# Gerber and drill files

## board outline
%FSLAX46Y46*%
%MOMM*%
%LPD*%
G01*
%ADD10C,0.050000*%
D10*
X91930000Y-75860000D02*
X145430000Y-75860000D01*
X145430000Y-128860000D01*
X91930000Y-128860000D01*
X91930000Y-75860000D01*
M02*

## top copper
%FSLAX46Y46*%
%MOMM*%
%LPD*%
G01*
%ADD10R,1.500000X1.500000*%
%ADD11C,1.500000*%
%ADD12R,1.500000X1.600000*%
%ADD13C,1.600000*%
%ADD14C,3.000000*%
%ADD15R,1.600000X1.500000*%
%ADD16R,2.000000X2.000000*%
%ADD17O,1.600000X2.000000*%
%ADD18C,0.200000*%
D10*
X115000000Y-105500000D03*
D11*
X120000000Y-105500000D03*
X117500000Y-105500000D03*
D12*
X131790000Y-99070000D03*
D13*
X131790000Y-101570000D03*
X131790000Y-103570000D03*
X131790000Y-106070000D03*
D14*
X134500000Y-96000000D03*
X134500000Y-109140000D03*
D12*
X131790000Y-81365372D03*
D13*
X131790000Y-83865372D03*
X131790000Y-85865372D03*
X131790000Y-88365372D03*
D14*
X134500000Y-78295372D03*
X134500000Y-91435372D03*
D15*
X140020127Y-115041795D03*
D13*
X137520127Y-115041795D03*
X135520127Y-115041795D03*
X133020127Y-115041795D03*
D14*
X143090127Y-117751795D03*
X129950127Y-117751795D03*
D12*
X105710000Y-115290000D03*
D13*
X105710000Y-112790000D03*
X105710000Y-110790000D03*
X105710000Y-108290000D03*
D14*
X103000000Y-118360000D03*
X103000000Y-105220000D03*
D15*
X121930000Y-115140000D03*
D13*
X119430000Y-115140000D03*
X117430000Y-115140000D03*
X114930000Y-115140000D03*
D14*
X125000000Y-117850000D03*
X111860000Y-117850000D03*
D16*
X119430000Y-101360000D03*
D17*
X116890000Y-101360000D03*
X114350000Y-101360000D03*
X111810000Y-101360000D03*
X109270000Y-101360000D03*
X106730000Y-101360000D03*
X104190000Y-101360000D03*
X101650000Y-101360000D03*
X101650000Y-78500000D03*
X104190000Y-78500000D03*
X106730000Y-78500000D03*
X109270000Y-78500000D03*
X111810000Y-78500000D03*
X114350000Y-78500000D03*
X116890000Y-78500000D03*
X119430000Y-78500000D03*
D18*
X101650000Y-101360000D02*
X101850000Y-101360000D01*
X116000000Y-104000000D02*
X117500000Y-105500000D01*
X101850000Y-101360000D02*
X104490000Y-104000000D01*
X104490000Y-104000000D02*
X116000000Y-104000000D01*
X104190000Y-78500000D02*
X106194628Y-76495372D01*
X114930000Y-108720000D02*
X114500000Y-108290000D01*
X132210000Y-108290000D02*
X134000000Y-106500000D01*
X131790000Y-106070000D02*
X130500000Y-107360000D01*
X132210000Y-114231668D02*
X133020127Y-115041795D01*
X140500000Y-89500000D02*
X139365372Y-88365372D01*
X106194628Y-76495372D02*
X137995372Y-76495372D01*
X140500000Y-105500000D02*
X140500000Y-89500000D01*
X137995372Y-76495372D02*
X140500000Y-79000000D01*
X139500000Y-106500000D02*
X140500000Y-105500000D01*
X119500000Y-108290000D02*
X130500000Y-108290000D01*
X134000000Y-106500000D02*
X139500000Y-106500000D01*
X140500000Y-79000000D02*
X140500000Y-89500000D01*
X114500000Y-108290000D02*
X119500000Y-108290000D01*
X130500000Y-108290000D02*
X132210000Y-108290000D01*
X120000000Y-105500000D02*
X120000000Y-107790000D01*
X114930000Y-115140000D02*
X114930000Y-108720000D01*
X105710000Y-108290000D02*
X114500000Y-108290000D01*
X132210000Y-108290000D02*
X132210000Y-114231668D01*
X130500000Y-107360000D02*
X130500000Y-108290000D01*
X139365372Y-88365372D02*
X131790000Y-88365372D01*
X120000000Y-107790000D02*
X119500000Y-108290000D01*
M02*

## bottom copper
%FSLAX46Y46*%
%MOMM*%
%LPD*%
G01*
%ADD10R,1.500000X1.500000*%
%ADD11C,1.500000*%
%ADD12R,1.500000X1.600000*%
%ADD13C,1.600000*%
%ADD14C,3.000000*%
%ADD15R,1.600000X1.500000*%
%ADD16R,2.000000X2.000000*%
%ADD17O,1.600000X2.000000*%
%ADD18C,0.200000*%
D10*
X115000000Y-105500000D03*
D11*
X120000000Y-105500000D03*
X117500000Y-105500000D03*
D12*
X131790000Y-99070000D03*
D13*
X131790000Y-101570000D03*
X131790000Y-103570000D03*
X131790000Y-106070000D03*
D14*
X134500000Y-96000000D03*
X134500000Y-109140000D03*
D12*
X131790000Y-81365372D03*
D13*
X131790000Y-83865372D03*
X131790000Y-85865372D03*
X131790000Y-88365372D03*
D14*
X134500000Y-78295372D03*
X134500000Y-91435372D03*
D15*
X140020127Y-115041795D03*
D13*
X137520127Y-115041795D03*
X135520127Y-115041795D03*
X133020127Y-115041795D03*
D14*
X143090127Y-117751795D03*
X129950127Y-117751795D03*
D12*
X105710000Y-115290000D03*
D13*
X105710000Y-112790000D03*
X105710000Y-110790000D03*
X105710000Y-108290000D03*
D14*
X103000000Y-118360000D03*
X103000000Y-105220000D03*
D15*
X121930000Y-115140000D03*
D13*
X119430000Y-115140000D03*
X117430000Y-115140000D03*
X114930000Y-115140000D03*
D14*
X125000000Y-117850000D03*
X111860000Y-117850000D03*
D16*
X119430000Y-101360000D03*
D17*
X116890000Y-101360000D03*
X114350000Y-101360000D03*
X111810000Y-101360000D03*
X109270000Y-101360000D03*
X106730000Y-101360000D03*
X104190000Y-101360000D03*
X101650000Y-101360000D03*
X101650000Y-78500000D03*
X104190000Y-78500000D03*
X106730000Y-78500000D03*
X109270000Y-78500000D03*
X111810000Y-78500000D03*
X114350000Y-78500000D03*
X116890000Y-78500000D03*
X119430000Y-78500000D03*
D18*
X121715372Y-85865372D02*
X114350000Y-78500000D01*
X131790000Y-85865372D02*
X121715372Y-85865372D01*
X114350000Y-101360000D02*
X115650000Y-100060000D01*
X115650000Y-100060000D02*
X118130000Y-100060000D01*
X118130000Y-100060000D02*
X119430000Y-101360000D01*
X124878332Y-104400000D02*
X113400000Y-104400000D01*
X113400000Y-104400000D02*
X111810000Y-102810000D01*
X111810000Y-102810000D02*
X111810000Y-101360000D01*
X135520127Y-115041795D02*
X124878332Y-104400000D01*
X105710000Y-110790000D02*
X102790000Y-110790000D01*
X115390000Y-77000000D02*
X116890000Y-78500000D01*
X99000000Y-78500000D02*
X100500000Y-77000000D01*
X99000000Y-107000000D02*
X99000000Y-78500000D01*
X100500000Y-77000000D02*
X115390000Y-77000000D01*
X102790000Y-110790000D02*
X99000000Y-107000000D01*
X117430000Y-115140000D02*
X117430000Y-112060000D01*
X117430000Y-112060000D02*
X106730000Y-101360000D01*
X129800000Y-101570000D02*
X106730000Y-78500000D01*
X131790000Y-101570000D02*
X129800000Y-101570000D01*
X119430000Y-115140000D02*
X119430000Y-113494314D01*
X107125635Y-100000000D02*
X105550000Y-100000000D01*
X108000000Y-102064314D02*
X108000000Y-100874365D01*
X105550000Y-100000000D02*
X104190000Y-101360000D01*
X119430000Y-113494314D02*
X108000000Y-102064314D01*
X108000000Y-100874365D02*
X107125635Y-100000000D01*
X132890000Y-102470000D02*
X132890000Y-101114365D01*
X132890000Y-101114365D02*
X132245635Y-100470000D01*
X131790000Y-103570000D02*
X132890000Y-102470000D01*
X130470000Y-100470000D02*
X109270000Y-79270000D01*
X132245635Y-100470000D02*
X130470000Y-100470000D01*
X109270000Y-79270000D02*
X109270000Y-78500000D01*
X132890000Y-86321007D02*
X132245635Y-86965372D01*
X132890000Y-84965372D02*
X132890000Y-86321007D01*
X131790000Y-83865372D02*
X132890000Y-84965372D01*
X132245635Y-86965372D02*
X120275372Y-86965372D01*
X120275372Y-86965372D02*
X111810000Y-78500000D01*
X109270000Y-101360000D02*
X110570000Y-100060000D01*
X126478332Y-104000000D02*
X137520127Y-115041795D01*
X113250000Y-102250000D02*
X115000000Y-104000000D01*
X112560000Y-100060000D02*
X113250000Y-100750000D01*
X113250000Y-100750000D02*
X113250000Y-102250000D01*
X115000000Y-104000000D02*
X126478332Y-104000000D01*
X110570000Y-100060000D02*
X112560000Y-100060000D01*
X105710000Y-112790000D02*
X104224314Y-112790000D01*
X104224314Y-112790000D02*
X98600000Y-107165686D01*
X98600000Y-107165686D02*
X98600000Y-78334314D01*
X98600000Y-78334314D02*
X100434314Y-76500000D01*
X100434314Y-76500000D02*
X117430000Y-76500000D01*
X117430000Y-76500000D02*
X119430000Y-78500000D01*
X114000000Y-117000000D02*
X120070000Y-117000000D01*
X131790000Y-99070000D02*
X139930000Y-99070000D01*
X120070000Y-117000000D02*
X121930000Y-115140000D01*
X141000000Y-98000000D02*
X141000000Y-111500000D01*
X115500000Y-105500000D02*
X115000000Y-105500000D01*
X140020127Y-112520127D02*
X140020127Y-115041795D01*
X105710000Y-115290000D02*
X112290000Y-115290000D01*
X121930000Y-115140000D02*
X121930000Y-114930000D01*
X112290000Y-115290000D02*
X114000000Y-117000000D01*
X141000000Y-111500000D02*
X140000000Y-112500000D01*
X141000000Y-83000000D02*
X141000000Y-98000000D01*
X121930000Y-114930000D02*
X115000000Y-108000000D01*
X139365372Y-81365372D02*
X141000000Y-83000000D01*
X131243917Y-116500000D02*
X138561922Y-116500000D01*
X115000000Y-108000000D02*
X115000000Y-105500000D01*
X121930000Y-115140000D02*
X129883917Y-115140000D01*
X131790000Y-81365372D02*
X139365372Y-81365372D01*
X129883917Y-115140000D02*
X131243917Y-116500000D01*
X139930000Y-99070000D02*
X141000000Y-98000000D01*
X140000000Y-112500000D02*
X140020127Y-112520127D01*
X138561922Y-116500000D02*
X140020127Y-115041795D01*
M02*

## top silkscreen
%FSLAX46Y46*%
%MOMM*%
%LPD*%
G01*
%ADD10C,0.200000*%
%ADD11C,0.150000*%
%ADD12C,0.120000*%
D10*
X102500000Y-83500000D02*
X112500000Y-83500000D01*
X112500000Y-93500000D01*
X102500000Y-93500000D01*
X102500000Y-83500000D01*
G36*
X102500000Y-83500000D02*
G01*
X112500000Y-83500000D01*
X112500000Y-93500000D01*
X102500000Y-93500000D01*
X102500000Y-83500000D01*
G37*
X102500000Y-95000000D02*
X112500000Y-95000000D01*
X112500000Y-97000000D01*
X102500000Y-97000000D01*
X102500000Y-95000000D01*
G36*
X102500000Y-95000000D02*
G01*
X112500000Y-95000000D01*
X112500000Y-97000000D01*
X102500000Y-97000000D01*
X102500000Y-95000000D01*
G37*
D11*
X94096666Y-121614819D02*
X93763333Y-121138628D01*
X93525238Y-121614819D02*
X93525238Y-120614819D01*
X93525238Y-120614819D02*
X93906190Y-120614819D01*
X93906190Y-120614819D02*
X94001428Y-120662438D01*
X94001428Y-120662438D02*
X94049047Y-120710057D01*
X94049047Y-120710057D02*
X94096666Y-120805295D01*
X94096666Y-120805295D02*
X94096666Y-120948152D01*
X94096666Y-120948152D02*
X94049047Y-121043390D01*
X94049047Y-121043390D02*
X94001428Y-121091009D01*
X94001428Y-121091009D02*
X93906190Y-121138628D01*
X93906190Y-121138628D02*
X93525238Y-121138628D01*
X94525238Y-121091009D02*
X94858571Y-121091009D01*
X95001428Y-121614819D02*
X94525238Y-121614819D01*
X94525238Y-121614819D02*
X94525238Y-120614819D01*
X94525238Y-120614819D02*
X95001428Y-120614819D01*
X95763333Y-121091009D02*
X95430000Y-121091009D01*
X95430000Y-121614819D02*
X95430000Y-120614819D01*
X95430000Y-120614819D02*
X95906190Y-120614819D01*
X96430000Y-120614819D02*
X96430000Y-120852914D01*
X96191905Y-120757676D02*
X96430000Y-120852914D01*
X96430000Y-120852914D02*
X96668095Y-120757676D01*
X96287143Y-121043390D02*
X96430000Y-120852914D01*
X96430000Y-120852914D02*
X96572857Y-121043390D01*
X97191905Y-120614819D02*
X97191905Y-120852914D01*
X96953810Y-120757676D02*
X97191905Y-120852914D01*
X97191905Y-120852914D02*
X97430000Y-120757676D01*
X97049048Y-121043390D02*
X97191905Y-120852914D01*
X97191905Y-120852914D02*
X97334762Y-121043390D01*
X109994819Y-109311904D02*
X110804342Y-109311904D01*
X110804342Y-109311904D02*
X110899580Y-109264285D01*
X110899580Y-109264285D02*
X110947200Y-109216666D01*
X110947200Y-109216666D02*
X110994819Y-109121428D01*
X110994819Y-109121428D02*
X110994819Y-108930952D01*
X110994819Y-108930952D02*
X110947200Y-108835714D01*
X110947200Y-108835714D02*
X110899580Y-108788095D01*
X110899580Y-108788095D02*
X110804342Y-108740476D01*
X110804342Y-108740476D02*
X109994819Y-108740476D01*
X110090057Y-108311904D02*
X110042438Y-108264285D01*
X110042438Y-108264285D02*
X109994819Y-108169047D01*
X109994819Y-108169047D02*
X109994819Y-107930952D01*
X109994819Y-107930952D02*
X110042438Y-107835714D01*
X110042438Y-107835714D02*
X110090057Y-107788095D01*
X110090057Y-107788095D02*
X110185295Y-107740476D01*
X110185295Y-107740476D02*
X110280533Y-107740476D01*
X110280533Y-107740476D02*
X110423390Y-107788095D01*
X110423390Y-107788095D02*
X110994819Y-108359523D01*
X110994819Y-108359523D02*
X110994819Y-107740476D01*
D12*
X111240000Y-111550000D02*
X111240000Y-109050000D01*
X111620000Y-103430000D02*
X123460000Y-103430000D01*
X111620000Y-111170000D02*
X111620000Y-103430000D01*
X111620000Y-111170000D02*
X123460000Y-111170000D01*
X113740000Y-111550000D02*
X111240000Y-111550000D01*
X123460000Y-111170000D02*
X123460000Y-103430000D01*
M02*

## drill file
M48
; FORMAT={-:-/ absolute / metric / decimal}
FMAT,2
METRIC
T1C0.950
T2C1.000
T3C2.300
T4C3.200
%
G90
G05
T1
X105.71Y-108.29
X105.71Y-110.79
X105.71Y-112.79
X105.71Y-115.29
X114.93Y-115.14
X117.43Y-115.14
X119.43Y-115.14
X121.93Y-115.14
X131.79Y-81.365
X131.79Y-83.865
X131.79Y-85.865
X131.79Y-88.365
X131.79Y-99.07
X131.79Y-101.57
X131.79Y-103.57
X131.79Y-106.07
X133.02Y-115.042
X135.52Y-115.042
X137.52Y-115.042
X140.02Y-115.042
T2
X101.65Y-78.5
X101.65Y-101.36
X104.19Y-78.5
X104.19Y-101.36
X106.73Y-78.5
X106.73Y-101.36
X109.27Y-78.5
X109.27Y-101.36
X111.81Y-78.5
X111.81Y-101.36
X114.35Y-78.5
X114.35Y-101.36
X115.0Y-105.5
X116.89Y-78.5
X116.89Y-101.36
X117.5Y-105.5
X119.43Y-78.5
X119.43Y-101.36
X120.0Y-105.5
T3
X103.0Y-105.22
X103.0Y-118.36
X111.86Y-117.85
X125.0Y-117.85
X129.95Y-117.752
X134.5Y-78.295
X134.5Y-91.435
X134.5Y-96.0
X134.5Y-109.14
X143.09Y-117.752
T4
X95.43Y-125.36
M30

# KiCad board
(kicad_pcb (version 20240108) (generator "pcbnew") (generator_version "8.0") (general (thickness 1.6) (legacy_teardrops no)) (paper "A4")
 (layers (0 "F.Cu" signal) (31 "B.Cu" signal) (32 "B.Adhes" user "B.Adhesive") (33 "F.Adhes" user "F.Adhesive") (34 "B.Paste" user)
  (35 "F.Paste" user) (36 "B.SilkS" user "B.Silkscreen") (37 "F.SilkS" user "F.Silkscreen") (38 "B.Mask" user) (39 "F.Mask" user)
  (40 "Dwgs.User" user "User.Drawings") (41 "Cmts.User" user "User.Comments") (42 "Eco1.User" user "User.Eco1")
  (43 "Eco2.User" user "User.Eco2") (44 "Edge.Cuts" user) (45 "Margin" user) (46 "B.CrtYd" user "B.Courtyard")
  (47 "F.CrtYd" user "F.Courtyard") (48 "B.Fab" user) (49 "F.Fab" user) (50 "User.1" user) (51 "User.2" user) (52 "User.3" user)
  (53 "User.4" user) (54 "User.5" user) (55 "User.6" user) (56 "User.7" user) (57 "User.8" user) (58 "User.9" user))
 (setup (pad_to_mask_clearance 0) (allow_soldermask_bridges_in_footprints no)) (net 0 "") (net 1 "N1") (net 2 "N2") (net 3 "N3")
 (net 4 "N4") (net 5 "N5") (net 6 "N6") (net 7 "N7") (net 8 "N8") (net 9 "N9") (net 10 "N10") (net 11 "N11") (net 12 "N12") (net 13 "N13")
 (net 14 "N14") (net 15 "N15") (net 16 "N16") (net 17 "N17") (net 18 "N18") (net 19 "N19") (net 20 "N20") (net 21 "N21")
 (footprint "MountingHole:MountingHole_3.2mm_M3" (layer "F.Cu") (at 95.43 125.36)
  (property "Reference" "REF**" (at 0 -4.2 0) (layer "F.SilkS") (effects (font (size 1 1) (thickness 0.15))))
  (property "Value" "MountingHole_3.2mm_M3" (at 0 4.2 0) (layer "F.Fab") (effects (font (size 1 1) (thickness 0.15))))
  (pad "" np_thru_hole circle (at 0 0) (size 3.2 3.2) (drill 3.2) (layers "*.Cu" "*.Mask")))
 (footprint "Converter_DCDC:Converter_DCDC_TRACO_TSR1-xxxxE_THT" (layer "F.Cu") (at 115 109 90)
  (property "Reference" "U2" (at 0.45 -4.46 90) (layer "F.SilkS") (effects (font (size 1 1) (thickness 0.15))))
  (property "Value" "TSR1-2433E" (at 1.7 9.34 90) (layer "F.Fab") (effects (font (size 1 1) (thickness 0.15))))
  (fp_line (start -2.55 -3.76) (end -0.05 -3.76) (stroke (width 0.12) (type solid)) (layer "F.SilkS"))
  (fp_line (start 5.57 -3.38) (end 5.57 8.46) (stroke (width 0.12) (type solid)) (layer "F.SilkS"))
  (fp_line (start -2.17 -3.38) (end 5.57 -3.38) (stroke (width 0.12) (type solid)) (layer "F.SilkS"))
  (fp_line (start -2.17 -3.38) (end -2.17 8.46) (stroke (width 0.12) (type solid)) (layer "F.SilkS"))
  (fp_line (start -2.55 -1.26) (end -2.55 -3.76) (stroke (width 0.12) (type solid)) (layer "F.SilkS"))
  (fp_line (start -2.17 8.46) (end 5.57 8.46) (stroke (width 0.12) (type solid)) (layer "F.SilkS"))
  (pad "1" thru_hole rect (at 3.5 0 90) (size 1.5 1.5) (drill 1) (layers "*.Cu" "*.Mask") (remove_unused_layers no) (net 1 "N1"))
  (pad "2" thru_hole circle (at 3.5 5 90) (size 1.5 1.5) (drill 1) (layers "*.Cu" "*.Mask") (remove_unused_layers no) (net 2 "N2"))
  (pad "3" thru_hole circle (at 3.5 2.5 90) (size 1.5 1.5) (drill 1) (layers "*.Cu" "*.Mask") (remove_unused_layers no) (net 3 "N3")))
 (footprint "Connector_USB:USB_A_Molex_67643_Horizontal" (layer "B.Cu") (at 131.79 99.07 -90)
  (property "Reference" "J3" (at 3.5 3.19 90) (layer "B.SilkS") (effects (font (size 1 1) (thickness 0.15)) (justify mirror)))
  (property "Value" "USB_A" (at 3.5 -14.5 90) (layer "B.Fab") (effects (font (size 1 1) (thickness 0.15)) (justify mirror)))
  (pad "1" thru_hole rect (at 0 0 270) (size 1.6 1.5) (drill 0.95) (layers "*.Cu" "*.Mask") (remove_unused_layers no) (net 1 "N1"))
  (pad "2" thru_hole circle (at 2.5 0 270) (size 1.6 1.6) (drill 0.95) (layers "*.Cu" "*.Mask") (remove_unused_layers no) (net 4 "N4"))
  (pad "3" thru_hole circle (at 4.5 0 270) (size 1.6 1.6) (drill 0.95) (layers "*.Cu" "*.Mask") (remove_unused_layers no) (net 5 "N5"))
  (pad "4" thru_hole circle (at 7 0 270) (size 1.6 1.6) (drill 0.95) (layers "*.Cu" "*.Mask") (remove_unused_layers no) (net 2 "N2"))
  (pad "5" thru_hole circle (at -3.07 -2.71 270) (size 3 3) (drill 2.3) (layers "*.Cu" "*.Mask") (remove_unused_layers no) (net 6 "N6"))
  (pad "5" thru_hole circle (at 10.07 -2.71 270) (size 3 3) (drill 2.3) (layers "*.Cu" "*.Mask") (remove_unused_layers no) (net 6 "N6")))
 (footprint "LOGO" (layer "B.Cu") (at 105 125.5 180)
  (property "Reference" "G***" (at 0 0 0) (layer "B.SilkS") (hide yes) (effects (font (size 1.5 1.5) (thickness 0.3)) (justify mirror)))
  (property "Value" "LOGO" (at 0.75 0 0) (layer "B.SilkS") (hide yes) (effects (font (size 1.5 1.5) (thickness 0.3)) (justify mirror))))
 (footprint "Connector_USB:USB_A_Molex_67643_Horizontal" (layer "B.Cu") (at 131.79 81.365372 -90)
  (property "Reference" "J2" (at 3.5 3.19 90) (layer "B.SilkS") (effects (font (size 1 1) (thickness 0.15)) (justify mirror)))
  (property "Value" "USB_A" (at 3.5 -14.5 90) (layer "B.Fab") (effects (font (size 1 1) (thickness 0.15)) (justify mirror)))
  (pad "1" thru_hole rect (at 0 0 270) (size 1.6 1.5) (drill 0.95) (layers "*.Cu" "*.Mask") (remove_unused_layers no) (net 1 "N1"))
  (pad "2" thru_hole circle (at 2.5 0 270) (size 1.6 1.6) (drill 0.95) (layers "*.Cu" "*.Mask") (remove_unused_layers no) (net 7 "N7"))
  (pad "3" thru_hole circle (at 4.5 0 270) (size 1.6 1.6) (drill 0.95) (layers "*.Cu" "*.Mask") (remove_unused_layers no) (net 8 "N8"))
  (pad "4" thru_hole circle (at 7 0 270) (size 1.6 1.6) (drill 0.95) (layers "*.Cu" "*.Mask") (remove_unused_layers no) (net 2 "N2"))
  (pad "5" thru_hole circle (at -3.07 -2.71 270) (size 3 3) (drill 2.3) (layers "*.Cu" "*.Mask") (remove_unused_layers no) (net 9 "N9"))
  (pad "5" thru_hole circle (at 10.07 -2.71 270) (size 3 3) (drill 2.3) (layers "*.Cu" "*.Mask") (remove_unused_layers no) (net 9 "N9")))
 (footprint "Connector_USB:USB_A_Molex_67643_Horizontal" (layer "B.Cu") (at 140.020127 115.041795 180)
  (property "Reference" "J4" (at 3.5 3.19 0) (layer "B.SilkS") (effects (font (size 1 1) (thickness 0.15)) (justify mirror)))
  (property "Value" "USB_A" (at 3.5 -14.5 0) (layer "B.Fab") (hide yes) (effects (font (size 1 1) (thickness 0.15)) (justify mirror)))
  (pad "1" thru_hole rect (at 0 0 180) (size 1.6 1.5) (drill 0.95) (layers "*.Cu" "*.Mask") (remove_unused_layers no) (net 1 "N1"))
  (pad "2" thru_hole circle (at 2.5 0 180) (size 1.6 1.6) (drill 0.95) (layers "*.Cu" "*.Mask") (remove_unused_layers no) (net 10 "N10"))
  (pad "3" thru_hole circle (at 4.5 0 180) (size 1.6 1.6) (drill 0.95) (layers "*.Cu" "*.Mask") (remove_unused_layers no) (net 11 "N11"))
  (pad "4" thru_hole circle (at 7 0 180) (size 1.6 1.6) (drill 0.95) (layers "*.Cu" "*.Mask") (remove_unused_layers no) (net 2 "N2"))
  (pad "5" thru_hole circle (at -3.07 -2.71 180) (size 3 3) (drill 2.3) (layers "*.Cu" "*.Mask") (remove_unused_layers no) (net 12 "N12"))
  (pad "5" thru_hole circle (at 10.07 -2.71 180) (size 3 3) (drill 2.3) (layers "*.Cu" "*.Mask") (remove_unused_layers no) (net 12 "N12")))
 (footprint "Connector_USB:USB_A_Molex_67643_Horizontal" (layer "B.Cu") (at 105.71 115.29 90)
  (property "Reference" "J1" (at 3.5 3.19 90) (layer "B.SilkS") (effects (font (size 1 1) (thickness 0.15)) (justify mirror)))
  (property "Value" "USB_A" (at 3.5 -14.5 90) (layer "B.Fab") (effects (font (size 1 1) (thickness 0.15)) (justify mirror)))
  (pad "1" thru_hole rect (at 0 0 90) (size 1.6 1.5) (drill 0.95) (layers "*.Cu" "*.Mask") (remove_unused_layers no) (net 1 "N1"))
  (pad "2" thru_hole circle (at 2.5 0 90) (size 1.6 1.6) (drill 0.95) (layers "*.Cu" "*.Mask") (remove_unused_layers no) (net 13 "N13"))
  (pad "3" thru_hole circle (at 4.5 0 90) (size 1.6 1.6) (drill 0.95) (layers "*.Cu" "*.Mask") (remove_unused_layers no) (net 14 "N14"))
  (pad "4" thru_hole circle (at 7 0 90) (size 1.6 1.6) (drill 0.95) (layers "*.Cu" "*.Mask") (remove_unused_layers no) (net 2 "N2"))
  (pad "5" thru_hole circle (at -3.07 -2.71 90) (size 3 3) (drill 2.3) (layers "*.Cu" "*.Mask") (remove_unused_layers no) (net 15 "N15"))
  (pad "5" thru_hole circle (at 10.07 -2.71 90) (size 3 3) (drill 2.3) (layers "*.Cu" "*.Mask") (remove_unused_layers no) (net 15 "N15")))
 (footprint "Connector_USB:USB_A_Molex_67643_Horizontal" (layer "B.Cu") (at 121.93 115.14 180)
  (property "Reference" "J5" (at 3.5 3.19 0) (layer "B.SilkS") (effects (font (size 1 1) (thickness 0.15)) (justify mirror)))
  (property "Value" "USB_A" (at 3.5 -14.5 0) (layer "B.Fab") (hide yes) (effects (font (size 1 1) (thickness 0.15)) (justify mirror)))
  (pad "1" thru_hole rect (at 0 0 180) (size 1.6 1.5) (drill 0.95) (layers "*.Cu" "*.Mask") (remove_unused_layers no) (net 1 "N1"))
  (pad "2" thru_hole circle (at 2.5 0 180) (size 1.6 1.6) (drill 0.95) (layers "*.Cu" "*.Mask") (remove_unused_layers no) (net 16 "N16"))
  (pad "3" thru_hole circle (at 4.5 0 180) (size 1.6 1.6) (drill 0.95) (layers "*.Cu" "*.Mask") (remove_unused_layers no) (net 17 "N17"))
  (pad "4" thru_hole circle (at 7 0 180) (size 1.6 1.6) (drill 0.95) (layers "*.Cu" "*.Mask") (remove_unused_layers no) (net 2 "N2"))
  (pad "5" thru_hole circle (at -3.07 -2.71 180) (size 3 3) (drill 2.3) (layers "*.Cu" "*.Mask") (remove_unused_layers no) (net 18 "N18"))
  (pad "5" thru_hole circle (at 10.07 -2.71 180) (size 3 3) (drill 2.3) (layers "*.Cu" "*.Mask") (remove_unused_layers no) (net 18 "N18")))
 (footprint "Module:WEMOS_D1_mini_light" (layer "B.Cu") (at 119.43 101.36 90)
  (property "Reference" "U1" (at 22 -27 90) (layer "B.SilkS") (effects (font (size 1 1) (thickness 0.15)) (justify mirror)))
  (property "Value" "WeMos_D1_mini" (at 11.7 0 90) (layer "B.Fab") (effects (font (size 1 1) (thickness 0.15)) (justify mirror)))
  (pad "1" thru_hole rect (at 0 0 90) (size 2 2) (drill 1) (layers "*.Cu" "*.Mask") (remove_unused_layers no) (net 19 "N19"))
  (pad "2" thru_hole oval (at 0 -2.54 90) (size 2 1.6) (drill 1) (layers "*.Cu" "*.Mask") (remove_unused_layers no) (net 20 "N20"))
  (pad "3" thru_hole oval (at 0 -5.08 90) (size 2 1.6) (drill 1) (layers "*.Cu" "*.Mask") (remove_unused_layers no) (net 19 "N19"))
  (pad "4" thru_hole oval (at 0 -7.62 90) (size 2 1.6) (drill 1) (layers "*.Cu" "*.Mask") (remove_unused_layers no) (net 11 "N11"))
  (pad "5" thru_hole oval (at 0 -10.16 90) (size 2 1.6) (drill 1) (layers "*.Cu" "*.Mask") (remove_unused_layers no) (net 10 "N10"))
  (pad "6" thru_hole oval (at 0 -12.7 90) (size 2 1.6) (drill 1) (layers "*.Cu" "*.Mask") (remove_unused_layers no) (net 17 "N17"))
  (pad "7" thru_hole oval (at 0 -15.24 90) (size 2 1.6) (drill 1) (layers "*.Cu" "*.Mask") (remove_unused_layers no) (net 16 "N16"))
  (pad "8" thru_hole oval (at 0 -17.78 90) (size 2 1.6) (drill 1) (layers "*.Cu" "*.Mask") (remove_unused_layers no) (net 3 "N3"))
  (pad "9" thru_hole oval (at 22.86 -17.78 90) (size 2 1.6) (drill 1) (layers "*.Cu" "*.Mask") (remove_unused_layers no) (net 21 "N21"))
  (pad "10" thru_hole oval (at 22.86 -15.24 90) (size 2 1.6) (drill 1) (layers "*.Cu" "*.Mask") (remove_unused_layers no) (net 2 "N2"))
  (pad "11" thru_hole oval (at 22.86 -12.7 90) (size 2 1.6) (drill 1) (layers "*.Cu" "*.Mask") (remove_unused_layers no) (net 4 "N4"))
  (pad "12" thru_hole oval (at 22.86 -10.16 90) (size 2 1.6) (drill 1) (layers "*.Cu" "*.Mask") (remove_unused_layers no) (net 5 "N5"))
  (pad "13" thru_hole oval (at 22.86 -7.62 90) (size 2 1.6) (drill 1) (layers "*.Cu" "*.Mask") (remove_unused_layers no) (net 7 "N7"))
  (pad "14" thru_hole oval (at 22.86 -5.08 90) (size 2 1.6) (drill 1) (layers "*.Cu" "*.Mask") (remove_unused_layers no) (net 8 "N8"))
  (pad "15" thru_hole oval (at 22.86 -2.54 90) (size 2 1.6) (drill 1) (layers "*.Cu" "*.Mask") (remove_unused_layers no) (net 14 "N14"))
  (pad "16" thru_hole oval (at 22.86 0 90) (size 2 1.6) (drill 1) (layers "*.Cu" "*.Mask") (remove_unused_layers no) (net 13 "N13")))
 (gr_rect (start 102.5 83.5) (end 112.5 93.5) (stroke (width 0.2) (type solid)) (fill solid) (layer "F.SilkS"))
 (gr_rect (start 102.5 95) (end 112.5 97) (stroke (width 0.2) (type solid)) (fill solid) (layer "F.SilkS"))
 (gr_rect (start 91.93 75.86) (end 145.43 128.86) (stroke (width 0.05) (type default)) (fill none) (layer "Edge.Cuts"))
 (segment (start 121.715372 85.865372) (end 114.35 78.5) (width 0.2) (layer "B.Cu") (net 8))
 (segment (start 131.79 85.865372) (end 121.715372 85.865372) (width 0.2) (layer "B.Cu") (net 8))
 (segment (start 114.35 101.36) (end 115.65 100.06) (width 0.2) (layer "B.Cu") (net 19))
 (segment (start 115.65 100.06) (end 118.13 100.06) (width 0.2) (layer "B.Cu") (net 19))
 (segment (start 118.13 100.06) (end 119.43 101.36) (width 0.2) (layer "B.Cu") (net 19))
 (segment (start 124.878332 104.4) (end 113.4 104.4) (width 0.2) (layer "B.Cu") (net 11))
 (segment (start 113.4 104.4) (end 111.81 102.81) (width 0.2) (layer "B.Cu") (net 11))
 (segment (start 111.81 102.81) (end 111.81 101.36) (width 0.2) (layer "B.Cu") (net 11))
 (segment (start 135.520127 115.041795) (end 124.878332 104.4) (width 0.2) (layer "B.Cu") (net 11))
 (segment (start 105.71 110.79) (end 102.79 110.79) (width 0.2) (layer "B.Cu") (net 14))
 (segment (start 115.39 77) (end 116.89 78.5) (width 0.2) (layer "B.Cu") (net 14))
 (segment (start 99 78.5) (end 100.5 77) (width 0.2) (layer "B.Cu") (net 14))
 (segment (start 99 107) (end 99 78.5) (width 0.2) (layer "B.Cu") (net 14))
 (segment (start 100.5 77) (end 115.39 77) (width 0.2) (layer "B.Cu") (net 14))
 (segment (start 102.79 110.79) (end 99 107) (width 0.2) (layer "B.Cu") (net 14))
 (segment (start 117.43 115.14) (end 117.43 112.06) (width 0.2) (layer "B.Cu") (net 17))
 (segment (start 117.43 112.06) (end 106.73 101.36) (width 0.2) (layer "B.Cu") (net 17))
 (segment (start 129.8 101.57) (end 106.73 78.5) (width 0.2) (layer "B.Cu") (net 4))
 (segment (start 131.79 101.57) (end 129.8 101.57) (width 0.2) (layer "B.Cu") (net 4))
 (segment (start 119.43 115.14) (end 119.43 113.494314) (width 0.2) (layer "B.Cu") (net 16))
 (segment (start 107.125635 100) (end 105.55 100) (width 0.2) (layer "B.Cu") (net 16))
 (segment (start 108 102.064314) (end 108 100.874365) (width 0.2) (layer "B.Cu") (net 16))
 (segment (start 105.55 100) (end 104.19 101.36) (width 0.2) (layer "B.Cu") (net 16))
 (segment (start 119.43 113.494314) (end 108 102.064314) (width 0.2) (layer "B.Cu") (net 16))
 (segment (start 108 100.874365) (end 107.125635 100) (width 0.2) (layer "B.Cu") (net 16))
 (segment (start 132.89 102.47) (end 132.89 101.114365) (width 0.2) (layer "B.Cu") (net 5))
 (segment (start 132.89 101.114365) (end 132.245635 100.47) (width 0.2) (layer "B.Cu") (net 5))
 (segment (start 131.79 103.57) (end 132.89 102.47) (width 0.2) (layer "B.Cu") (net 5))
 (segment (start 130.47 100.47) (end 109.27 79.27) (width 0.2) (layer "B.Cu") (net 5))
 (segment (start 132.245635 100.47) (end 130.47 100.47) (width 0.2) (layer "B.Cu") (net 5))
 (segment (start 109.27 79.27) (end 109.27 78.5) (width 0.2) (layer "B.Cu") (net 5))
 (segment (start 132.89 86.321007) (end 132.245635 86.965372) (width 0.2) (layer "B.Cu") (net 7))
 (segment (start 132.89 84.965372) (end 132.89 86.321007) (width 0.2) (layer "B.Cu") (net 7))
 (segment (start 131.79 83.865372) (end 132.89 84.965372) (width 0.2) (layer "B.Cu") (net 7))
 (segment (start 132.245635 86.965372) (end 120.275372 86.965372) (width 0.2) (layer "B.Cu") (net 7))
 (segment (start 120.275372 86.965372) (end 111.81 78.5) (width 0.2) (layer "B.Cu") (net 7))
 (segment (start 101.65 101.36) (end 101.85 101.36) (width 0.2) (layer "F.Cu") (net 3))
 (segment (start 116 104) (end 117.5 105.5) (width 0.2) (layer "F.Cu") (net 3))
 (segment (start 101.85 101.36) (end 104.49 104) (width 0.2) (layer "F.Cu") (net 3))
 (segment (start 104.49 104) (end 116 104) (width 0.2) (layer "F.Cu") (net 3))
 (segment (start 109.27 101.36) (end 110.57 100.06) (width 0.2) (layer "B.Cu") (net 10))
 (segment (start 126.478332 104) (end 137.520127 115.041795) (width 0.2) (layer "B.Cu") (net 10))
 (segment (start 113.25 102.25) (end 115 104) (width 0.2) (layer "B.Cu") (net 10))
 (segment (start 112.56 100.06) (end 113.25 100.75) (width 0.2) (layer "B.Cu") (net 10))
 (segment (start 113.25 100.75) (end 113.25 102.25) (width 0.2) (layer "B.Cu") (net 10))
 (segment (start 115 104) (end 126.478332 104) (width 0.2) (layer "B.Cu") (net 10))
 (segment (start 110.57 100.06) (end 112.56 100.06) (width 0.2) (layer "B.Cu") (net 10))
 (segment (start 105.71 112.79) (end 104.224314 112.79) (width 0.2) (layer "B.Cu") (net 13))
 (segment (start 104.224314 112.79) (end 98.6 107.165686) (width 0.2) (layer "B.Cu") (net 13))
 (segment (start 98.6 107.165686) (end 98.6 78.334314) (width 0.2) (layer "B.Cu") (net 13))
 (segment (start 98.6 78.334314) (end 100.434314 76.5) (width 0.2) (layer "B.Cu") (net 13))
 (segment (start 100.434314 76.5) (end 117.43 76.5) (width 0.2) (layer "B.Cu") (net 13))
 (segment (start 117.43 76.5) (end 119.43 78.5) (width 0.2) (layer "B.Cu") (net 13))
 (segment (start 114 117) (end 120.07 117) (width 0.2) (layer "B.Cu") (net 1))
 (segment (start 131.79 99.07) (end 139.93 99.07) (width 0.2) (layer "B.Cu") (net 1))
 (segment (start 120.07 117) (end 121.93 115.14) (width 0.2) (layer "B.Cu") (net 1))
 (segment (start 141 98) (end 141 111.5) (width 0.2) (layer "B.Cu") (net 1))
 (segment (start 115.5 105.5) (end 115 105.5) (width 0.2) (layer "B.Cu") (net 1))
 (segment (start 140.020127 112.520127) (end 140.020127 115.041795) (width 0.2) (layer "B.Cu") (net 1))
 (segment (start 105.71 115.29) (end 112.29 115.29) (width 0.2) (layer "B.Cu") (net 1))
 (segment (start 121.93 115.14) (end 121.93 114.93) (width 0.2) (layer "B.Cu") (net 1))
 (segment (start 112.29 115.29) (end 114 117) (width 0.2) (layer "B.Cu") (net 1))
 (segment (start 141 111.5) (end 140 112.5) (width 0.2) (layer "B.Cu") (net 1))
 (segment (start 141 83) (end 141 98) (width 0.2) (layer "B.Cu") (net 1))
 (segment (start 121.93 114.93) (end 115 108) (width 0.2) (layer "B.Cu") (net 1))
 (segment (start 139.365372 81.365372) (end 141 83) (width 0.2) (layer "B.Cu") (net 1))
 (segment (start 131.243917 116.5) (end 138.561922 116.5) (width 0.2) (layer "B.Cu") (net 1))
 (segment (start 115 108) (end 115 105.5) (width 0.2) (layer "B.Cu") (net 1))
 (segment (start 121.93 115.14) (end 129.883917 115.14) (width 0.2) (layer "B.Cu") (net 1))
 (segment (start 131.79 81.365372) (end 139.365372 81.365372) (width 0.2) (layer "B.Cu") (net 1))
 (segment (start 129.883917 115.14) (end 131.243917 116.5) (width 0.2) (layer "B.Cu") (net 1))
 (segment (start 139.93 99.07) (end 141 98) (width 0.2) (layer "B.Cu") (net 1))
 (segment (start 140 112.5) (end 140.020127 112.520127) (width 0.2) (layer "B.Cu") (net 1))
 (segment (start 138.561922 116.5) (end 140.020127 115.041795) (width 0.2) (layer "B.Cu") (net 1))
 (segment (start 104.19 78.5) (end 106.194628 76.495372) (width 0.2) (layer "F.Cu") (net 2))
 (segment (start 114.93 108.72) (end 114.5 108.29) (width 0.2) (layer "F.Cu") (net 2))
 (segment (start 132.21 108.29) (end 134 106.5) (width 0.2) (layer "F.Cu") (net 2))
 (segment (start 131.79 106.07) (end 130.5 107.36) (width 0.2) (layer "F.Cu") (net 2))
 (segment (start 132.21 114.231668) (end 133.020127 115.041795) (width 0.2) (layer "F.Cu") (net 2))
 (segment (start 140.5 89.5) (end 139.365372 88.365372) (width 0.2) (layer "F.Cu") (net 2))
 (segment (start 106.194628 76.495372) (end 137.995372 76.495372) (width 0.2) (layer "F.Cu") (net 2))
 (segment (start 140.5 105.5) (end 140.5 89.5) (width 0.2) (layer "F.Cu") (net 2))
 (segment (start 137.995372 76.495372) (end 140.5 79) (width 0.2) (layer "F.Cu") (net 2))
 (segment (start 139.5 106.5) (end 140.5 105.5) (width 0.2) (layer "F.Cu") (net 2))
 (segment (start 119.5 108.29) (end 130.5 108.29) (width 0.2) (layer "F.Cu") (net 2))
 (segment (start 134 106.5) (end 139.5 106.5) (width 0.2) (layer "F.Cu") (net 2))
 (segment (start 140.5 79) (end 140.5 89.5) (width 0.2) (layer "F.Cu") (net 2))
 (segment (start 114.5 108.29) (end 119.5 108.29) (width 0.2) (layer "F.Cu") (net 2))
 (segment (start 130.5 108.29) (end 132.21 108.29) (width 0.2) (layer "F.Cu") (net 2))
 (segment (start 120 105.5) (end 120 107.79) (width 0.2) (layer "F.Cu") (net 2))
 (segment (start 114.93 115.14) (end 114.93 108.72) (width 0.2) (layer "F.Cu") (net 2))
 (segment (start 105.71 108.29) (end 114.5 108.29) (width 0.2) (layer "F.Cu") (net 2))
 (segment (start 132.21 108.29) (end 132.21 114.231668) (width 0.2) (layer "F.Cu") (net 2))
 (segment (start 130.5 107.36) (end 130.5 108.29) (width 0.2) (layer "F.Cu") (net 2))
 (segment (start 139.365372 88.365372) (end 131.79 88.365372) (width 0.2) (layer "F.Cu") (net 2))
 (segment (start 120 107.79) (end 119.5 108.29) (width 0.2) (layer "F.Cu") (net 2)))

